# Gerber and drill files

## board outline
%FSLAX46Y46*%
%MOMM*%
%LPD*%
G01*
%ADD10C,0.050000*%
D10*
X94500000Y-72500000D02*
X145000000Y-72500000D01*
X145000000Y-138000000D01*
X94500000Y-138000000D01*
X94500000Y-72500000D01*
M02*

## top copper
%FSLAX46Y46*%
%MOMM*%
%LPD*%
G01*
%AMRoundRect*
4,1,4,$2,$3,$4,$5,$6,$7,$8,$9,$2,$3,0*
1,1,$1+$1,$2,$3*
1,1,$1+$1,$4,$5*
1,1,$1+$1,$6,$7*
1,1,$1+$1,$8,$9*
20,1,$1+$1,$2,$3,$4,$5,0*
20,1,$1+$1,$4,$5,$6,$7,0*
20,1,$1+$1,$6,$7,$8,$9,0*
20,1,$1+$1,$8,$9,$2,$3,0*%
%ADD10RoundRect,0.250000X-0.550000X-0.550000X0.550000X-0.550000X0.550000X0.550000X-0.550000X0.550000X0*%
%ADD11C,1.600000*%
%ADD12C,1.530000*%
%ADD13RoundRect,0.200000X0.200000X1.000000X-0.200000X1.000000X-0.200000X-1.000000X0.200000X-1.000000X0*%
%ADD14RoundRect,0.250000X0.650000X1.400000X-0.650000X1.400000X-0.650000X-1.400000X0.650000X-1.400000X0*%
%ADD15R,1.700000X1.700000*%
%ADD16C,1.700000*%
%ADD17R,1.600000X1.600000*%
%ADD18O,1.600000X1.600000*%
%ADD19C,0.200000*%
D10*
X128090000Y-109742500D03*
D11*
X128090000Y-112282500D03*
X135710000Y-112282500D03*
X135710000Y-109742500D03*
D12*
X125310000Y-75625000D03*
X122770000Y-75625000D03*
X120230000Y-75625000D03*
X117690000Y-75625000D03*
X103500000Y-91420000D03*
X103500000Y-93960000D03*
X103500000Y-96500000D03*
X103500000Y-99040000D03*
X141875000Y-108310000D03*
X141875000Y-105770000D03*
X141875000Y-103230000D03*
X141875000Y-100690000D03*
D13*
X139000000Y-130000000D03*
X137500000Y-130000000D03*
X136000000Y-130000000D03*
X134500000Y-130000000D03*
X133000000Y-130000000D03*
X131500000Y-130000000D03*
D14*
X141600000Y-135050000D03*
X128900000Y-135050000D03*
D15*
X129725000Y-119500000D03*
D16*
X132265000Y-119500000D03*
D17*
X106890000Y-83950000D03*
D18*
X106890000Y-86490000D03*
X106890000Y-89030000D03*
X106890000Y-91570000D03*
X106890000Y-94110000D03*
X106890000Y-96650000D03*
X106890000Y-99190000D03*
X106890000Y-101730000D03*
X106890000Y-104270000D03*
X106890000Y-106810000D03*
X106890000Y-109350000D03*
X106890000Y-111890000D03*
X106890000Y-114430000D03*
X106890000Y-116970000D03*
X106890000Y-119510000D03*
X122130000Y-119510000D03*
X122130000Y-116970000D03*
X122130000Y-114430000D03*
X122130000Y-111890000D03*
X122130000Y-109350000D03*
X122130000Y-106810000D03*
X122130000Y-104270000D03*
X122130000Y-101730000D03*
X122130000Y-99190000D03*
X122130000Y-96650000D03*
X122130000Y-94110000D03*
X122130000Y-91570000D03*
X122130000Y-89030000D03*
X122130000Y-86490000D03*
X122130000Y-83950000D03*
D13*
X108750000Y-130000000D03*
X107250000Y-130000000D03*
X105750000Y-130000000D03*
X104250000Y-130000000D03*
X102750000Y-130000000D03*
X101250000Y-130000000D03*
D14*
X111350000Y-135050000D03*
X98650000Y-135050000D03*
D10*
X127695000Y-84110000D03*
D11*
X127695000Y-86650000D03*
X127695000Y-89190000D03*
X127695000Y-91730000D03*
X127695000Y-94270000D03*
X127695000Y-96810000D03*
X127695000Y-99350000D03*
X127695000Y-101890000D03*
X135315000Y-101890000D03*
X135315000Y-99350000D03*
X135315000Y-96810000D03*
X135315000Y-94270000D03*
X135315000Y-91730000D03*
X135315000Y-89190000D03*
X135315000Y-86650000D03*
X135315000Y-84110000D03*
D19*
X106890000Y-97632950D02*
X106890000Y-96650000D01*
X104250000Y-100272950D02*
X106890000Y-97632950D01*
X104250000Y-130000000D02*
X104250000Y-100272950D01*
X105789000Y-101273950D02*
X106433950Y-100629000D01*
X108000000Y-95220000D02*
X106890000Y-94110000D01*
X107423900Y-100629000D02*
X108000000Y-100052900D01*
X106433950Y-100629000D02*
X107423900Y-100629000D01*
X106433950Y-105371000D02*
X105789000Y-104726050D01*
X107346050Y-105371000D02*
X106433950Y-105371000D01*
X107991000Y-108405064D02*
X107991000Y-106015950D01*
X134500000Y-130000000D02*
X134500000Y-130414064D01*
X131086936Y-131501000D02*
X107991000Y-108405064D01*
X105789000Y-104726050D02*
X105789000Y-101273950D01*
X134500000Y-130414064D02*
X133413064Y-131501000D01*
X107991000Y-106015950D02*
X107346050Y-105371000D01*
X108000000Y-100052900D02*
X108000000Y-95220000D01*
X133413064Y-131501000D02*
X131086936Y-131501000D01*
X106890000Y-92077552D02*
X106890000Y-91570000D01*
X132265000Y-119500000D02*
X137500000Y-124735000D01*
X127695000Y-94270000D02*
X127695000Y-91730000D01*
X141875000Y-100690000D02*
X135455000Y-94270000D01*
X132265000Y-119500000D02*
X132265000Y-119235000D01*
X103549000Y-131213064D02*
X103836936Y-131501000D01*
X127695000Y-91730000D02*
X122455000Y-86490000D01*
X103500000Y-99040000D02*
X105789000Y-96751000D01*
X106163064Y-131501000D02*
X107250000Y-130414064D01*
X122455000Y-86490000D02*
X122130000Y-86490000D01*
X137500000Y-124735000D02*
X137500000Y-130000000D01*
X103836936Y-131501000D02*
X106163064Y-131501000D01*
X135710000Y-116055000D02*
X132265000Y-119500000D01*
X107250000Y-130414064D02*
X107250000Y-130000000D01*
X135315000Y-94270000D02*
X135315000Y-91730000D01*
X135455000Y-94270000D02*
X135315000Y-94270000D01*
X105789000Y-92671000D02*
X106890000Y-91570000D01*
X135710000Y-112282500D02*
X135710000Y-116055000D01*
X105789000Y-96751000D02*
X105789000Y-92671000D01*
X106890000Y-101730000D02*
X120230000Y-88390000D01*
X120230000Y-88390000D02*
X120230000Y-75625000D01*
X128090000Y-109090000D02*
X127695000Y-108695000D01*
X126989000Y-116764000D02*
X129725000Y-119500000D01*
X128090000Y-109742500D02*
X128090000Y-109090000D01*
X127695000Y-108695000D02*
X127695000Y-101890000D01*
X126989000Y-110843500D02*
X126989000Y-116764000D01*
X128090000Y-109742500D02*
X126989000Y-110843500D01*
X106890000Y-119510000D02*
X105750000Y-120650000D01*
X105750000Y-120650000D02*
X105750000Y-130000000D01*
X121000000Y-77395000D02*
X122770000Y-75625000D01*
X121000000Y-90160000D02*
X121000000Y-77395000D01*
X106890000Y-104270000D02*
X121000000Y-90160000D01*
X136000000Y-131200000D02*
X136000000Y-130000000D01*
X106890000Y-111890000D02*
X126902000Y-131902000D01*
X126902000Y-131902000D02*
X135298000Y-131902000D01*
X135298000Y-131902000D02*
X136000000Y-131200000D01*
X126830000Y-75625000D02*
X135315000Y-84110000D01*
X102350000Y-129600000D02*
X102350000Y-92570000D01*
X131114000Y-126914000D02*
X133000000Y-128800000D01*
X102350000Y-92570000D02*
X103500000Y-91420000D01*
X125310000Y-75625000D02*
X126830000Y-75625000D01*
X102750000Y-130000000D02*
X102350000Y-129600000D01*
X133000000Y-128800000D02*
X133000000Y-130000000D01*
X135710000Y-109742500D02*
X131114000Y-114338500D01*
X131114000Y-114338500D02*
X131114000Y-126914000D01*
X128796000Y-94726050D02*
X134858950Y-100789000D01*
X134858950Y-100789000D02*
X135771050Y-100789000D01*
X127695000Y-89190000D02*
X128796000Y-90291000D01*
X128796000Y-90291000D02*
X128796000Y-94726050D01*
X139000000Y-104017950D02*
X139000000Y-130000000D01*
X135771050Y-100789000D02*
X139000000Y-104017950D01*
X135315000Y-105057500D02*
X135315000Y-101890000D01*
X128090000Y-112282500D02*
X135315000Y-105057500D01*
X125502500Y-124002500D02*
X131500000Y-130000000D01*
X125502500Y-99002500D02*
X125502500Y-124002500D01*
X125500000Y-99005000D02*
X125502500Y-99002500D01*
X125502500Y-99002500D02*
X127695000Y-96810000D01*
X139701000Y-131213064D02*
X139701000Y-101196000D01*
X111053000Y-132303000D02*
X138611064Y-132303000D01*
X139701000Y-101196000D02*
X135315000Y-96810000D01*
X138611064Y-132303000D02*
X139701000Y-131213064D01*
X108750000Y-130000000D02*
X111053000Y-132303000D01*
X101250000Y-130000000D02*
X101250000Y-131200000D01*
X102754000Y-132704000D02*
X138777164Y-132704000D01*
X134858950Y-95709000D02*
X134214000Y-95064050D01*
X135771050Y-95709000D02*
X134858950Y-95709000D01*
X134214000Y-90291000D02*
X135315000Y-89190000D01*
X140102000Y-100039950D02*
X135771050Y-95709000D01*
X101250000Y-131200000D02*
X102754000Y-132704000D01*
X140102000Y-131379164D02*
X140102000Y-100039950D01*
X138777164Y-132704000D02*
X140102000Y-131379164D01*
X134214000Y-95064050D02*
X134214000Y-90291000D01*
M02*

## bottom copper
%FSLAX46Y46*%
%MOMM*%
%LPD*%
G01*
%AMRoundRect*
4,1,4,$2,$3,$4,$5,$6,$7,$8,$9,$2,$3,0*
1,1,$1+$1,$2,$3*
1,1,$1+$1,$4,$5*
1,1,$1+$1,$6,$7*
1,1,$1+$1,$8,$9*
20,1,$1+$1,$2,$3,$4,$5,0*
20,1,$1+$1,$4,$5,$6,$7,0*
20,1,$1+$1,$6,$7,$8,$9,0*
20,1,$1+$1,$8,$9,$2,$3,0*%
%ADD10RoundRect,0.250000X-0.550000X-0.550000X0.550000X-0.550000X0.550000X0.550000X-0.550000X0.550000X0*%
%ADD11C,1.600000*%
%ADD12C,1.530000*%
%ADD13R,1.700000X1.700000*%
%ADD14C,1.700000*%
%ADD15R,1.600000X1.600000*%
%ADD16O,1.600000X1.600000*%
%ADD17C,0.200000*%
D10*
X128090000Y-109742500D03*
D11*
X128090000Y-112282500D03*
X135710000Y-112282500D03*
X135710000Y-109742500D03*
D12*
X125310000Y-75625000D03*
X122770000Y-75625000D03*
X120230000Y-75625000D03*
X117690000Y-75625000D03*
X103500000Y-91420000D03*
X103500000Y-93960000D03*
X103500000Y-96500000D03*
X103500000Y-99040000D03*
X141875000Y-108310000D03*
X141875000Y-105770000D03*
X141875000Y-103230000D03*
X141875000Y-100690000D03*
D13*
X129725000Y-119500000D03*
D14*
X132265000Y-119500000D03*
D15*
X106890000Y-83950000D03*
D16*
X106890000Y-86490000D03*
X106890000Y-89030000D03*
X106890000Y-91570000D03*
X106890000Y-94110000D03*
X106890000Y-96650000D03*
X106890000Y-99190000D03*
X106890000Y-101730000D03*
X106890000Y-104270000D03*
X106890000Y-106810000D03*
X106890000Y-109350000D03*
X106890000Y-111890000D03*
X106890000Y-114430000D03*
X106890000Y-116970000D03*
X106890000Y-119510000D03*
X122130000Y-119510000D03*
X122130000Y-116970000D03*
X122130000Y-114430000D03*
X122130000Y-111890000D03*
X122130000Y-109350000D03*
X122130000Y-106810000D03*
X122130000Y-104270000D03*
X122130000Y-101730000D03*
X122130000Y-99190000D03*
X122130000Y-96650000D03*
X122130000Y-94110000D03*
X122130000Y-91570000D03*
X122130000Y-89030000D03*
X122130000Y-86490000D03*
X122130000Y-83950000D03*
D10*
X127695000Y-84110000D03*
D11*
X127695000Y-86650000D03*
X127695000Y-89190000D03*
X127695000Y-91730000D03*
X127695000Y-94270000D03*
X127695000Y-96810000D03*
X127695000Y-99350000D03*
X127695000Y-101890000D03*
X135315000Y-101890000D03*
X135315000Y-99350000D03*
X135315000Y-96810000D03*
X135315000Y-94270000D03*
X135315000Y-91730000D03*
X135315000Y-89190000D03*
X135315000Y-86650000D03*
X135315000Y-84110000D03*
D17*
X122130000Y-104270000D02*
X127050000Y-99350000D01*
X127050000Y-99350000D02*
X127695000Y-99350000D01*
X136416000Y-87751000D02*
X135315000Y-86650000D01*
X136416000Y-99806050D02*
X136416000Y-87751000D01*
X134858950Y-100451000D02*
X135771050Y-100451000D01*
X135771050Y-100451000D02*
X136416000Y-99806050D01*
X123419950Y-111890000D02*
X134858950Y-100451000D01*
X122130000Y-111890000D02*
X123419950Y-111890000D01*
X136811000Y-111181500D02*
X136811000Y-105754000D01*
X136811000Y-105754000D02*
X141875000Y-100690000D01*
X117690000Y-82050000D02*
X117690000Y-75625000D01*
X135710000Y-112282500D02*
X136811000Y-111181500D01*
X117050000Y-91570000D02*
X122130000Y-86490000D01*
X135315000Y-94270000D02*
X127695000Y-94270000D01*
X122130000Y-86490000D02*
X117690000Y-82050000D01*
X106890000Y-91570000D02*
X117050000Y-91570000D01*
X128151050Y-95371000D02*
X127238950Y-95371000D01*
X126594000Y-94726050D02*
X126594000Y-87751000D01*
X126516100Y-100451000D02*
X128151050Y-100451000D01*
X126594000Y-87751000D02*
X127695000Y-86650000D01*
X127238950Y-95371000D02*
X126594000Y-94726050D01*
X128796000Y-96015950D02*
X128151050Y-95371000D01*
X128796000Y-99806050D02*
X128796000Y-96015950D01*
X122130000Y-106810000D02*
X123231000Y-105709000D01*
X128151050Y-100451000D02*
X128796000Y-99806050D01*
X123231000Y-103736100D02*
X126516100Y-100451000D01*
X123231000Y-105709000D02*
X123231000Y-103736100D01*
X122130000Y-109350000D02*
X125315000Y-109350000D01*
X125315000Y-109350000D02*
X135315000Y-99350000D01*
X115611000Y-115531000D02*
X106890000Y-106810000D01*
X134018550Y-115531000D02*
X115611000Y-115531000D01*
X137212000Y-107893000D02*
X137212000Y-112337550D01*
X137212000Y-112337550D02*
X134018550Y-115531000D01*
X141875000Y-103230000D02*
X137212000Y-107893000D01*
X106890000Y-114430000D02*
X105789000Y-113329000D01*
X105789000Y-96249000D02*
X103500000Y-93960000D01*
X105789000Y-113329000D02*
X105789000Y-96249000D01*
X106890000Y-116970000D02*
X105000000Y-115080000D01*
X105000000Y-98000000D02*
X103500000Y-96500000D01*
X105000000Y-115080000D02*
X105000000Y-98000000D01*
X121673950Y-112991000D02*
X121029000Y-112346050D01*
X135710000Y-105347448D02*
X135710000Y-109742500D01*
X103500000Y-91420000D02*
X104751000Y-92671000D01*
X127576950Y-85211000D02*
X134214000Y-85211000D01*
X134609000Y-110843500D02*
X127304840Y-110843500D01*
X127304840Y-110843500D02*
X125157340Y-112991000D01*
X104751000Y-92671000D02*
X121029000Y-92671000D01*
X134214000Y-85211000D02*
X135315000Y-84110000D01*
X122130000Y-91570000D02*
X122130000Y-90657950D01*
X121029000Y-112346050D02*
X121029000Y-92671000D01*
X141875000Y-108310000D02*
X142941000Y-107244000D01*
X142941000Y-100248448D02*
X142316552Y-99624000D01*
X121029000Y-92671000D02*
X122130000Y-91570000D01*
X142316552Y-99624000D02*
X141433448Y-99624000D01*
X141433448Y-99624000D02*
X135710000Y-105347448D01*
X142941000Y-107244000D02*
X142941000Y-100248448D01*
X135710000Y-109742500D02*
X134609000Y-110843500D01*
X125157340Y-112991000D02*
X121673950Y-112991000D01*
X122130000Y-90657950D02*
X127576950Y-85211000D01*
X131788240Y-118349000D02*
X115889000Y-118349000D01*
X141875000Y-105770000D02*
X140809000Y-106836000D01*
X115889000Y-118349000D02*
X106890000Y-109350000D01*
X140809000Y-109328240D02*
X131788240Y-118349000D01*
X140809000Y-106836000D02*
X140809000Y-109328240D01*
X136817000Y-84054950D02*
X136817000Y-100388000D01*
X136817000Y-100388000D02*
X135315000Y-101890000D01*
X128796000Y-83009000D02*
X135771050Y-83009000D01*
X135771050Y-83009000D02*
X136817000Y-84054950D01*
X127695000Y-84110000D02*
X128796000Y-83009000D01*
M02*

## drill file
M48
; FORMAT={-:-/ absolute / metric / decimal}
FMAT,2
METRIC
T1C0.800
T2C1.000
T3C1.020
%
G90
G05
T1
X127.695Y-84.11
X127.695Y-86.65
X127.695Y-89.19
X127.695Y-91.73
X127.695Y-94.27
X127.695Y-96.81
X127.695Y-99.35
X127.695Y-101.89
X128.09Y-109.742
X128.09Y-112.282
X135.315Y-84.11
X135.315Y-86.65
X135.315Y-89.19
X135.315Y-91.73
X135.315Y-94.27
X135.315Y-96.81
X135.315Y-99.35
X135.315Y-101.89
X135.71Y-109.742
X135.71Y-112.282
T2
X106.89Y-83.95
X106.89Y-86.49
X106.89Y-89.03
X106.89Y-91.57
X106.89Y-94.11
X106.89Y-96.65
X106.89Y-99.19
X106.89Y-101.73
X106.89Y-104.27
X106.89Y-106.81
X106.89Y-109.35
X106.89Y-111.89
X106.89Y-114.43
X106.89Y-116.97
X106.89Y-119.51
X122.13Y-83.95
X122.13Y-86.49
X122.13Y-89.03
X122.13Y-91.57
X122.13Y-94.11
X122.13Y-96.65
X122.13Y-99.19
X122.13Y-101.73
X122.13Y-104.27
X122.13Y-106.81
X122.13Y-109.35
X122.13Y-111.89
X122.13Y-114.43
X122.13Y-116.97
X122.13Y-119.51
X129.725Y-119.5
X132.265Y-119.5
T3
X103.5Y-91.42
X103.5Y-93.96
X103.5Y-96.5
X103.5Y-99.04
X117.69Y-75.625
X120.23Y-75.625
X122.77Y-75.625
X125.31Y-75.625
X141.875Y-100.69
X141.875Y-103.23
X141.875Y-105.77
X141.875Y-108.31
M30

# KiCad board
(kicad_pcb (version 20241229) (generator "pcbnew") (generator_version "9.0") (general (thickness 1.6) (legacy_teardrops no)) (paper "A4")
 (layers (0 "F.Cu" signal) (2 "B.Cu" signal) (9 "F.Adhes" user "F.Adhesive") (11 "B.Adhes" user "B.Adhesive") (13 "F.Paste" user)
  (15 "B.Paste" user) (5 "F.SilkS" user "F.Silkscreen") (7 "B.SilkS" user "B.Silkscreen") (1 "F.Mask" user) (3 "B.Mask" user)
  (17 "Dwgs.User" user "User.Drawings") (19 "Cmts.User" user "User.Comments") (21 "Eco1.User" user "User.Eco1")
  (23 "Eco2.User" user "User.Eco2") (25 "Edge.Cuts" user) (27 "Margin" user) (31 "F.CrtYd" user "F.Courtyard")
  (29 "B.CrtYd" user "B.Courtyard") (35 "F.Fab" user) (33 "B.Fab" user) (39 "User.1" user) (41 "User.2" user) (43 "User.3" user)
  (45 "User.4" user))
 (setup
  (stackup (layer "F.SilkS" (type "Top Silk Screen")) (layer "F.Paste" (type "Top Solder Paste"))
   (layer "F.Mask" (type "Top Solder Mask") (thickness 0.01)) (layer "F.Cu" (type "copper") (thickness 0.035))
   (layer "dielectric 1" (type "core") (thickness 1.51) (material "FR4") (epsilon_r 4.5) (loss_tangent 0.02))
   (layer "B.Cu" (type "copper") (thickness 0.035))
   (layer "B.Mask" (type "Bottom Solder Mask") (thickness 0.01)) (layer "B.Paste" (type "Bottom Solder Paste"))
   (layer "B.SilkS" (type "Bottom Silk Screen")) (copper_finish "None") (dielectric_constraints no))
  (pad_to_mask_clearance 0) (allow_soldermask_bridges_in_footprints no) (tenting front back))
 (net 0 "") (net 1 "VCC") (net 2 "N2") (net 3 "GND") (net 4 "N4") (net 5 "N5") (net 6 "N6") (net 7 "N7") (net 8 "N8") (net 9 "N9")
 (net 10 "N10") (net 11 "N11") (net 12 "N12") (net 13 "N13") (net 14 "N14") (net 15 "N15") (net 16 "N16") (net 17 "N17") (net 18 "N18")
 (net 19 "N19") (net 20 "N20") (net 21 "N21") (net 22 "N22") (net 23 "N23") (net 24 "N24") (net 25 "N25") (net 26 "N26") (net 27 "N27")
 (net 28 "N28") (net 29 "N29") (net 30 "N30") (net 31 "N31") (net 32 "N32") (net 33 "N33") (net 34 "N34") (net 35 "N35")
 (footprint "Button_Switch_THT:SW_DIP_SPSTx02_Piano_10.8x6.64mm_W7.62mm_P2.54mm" (layer "F.Cu") (at 128.09 109.7425)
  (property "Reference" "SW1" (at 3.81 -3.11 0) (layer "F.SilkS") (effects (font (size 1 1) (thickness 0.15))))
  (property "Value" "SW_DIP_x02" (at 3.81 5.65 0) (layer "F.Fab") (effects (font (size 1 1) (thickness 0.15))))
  (pad "1" thru_hole roundrect (at 0 0) (size 1.6 1.6) (drill 0.8) (layers "*.Cu" "*.Mask") (remove_unused_layers no)
   (roundrect_rratio 0.15625) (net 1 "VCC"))
  (pad "2" thru_hole circle (at 0 2.54) (size 1.6 1.6) (drill 0.8) (layers "*.Cu" "*.Mask") (remove_unused_layers no) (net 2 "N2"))
  (pad "3" thru_hole circle (at 7.62 2.54) (size 1.6 1.6) (drill 0.8) (layers "*.Cu" "*.Mask") (remove_unused_layers no) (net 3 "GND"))
  (pad "4" thru_hole circle (at 7.62 0) (size 1.6 1.6) (drill 0.8) (layers "*.Cu" "*.Mask") (remove_unused_layers no) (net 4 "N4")))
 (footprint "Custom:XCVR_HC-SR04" (layer "F.Cu") (at 121.5 75.625 180)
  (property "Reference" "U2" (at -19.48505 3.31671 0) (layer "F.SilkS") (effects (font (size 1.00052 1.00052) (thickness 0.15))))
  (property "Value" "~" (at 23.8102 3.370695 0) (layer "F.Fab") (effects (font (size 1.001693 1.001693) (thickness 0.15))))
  (pad "1" thru_hole circle (at -3.81 0 180) (size 1.53 1.53) (drill 1.02) (layers "*.Cu" "*.Mask") (remove_unused_layers no) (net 4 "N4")
   (solder_mask_margin 0.102))
  (pad "2" thru_hole circle (at -1.27 0 180) (size 1.53 1.53) (drill 1.02) (layers "*.Cu" "*.Mask") (remove_unused_layers no) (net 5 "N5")
   (solder_mask_margin 0.102))
  (pad "3" thru_hole circle (at 1.27 0 180) (size 1.53 1.53) (drill 1.02) (layers "*.Cu" "*.Mask") (remove_unused_layers no) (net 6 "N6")
   (solder_mask_margin 0.102))
  (pad "4" thru_hole circle (at 3.81 0 180) (size 1.53 1.53) (drill 1.02) (layers "*.Cu" "*.Mask") (remove_unused_layers no) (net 3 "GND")
   (solder_mask_margin 0.102)))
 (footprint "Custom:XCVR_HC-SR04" (layer "F.Cu") (at 103.5 95.23 -90)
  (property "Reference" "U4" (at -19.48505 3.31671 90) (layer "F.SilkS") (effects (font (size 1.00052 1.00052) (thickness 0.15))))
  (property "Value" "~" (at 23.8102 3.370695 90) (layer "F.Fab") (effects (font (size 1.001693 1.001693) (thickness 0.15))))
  (pad "1" thru_hole circle (at -3.81 0 270) (size 1.53 1.53) (drill 1.02) (layers "*.Cu" "*.Mask") (remove_unused_layers no) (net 4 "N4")
   (solder_mask_margin 0.102))
  (pad "2" thru_hole circle (at -1.27 0 270) (size 1.53 1.53) (drill 1.02) (layers "*.Cu" "*.Mask") (remove_unused_layers no) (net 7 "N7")
   (solder_mask_margin 0.102))
  (pad "3" thru_hole circle (at 1.27 0 270) (size 1.53 1.53) (drill 1.02) (layers "*.Cu" "*.Mask") (remove_unused_layers no) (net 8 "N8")
   (solder_mask_margin 0.102))
  (pad "4" thru_hole circle (at 3.81 0 270) (size 1.53 1.53) (drill 1.02) (layers "*.Cu" "*.Mask") (remove_unused_layers no) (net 3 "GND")
   (solder_mask_margin 0.102)))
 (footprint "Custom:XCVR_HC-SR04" (layer "F.Cu") (at 141.875 104.5 90)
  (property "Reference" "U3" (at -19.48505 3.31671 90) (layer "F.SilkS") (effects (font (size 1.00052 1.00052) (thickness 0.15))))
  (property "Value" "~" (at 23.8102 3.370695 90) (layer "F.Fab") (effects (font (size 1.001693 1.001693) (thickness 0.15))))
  (pad "1" thru_hole circle (at -3.81 0 90) (size 1.53 1.53) (drill 1.02) (layers "*.Cu" "*.Mask") (remove_unused_layers no) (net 4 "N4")
   (solder_mask_margin 0.102))
  (pad "2" thru_hole circle (at -1.27 0 90) (size 1.53 1.53) (drill 1.02) (layers "*.Cu" "*.Mask") (remove_unused_layers no) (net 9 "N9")
   (solder_mask_margin 0.102))
  (pad "3" thru_hole circle (at 1.27 0 90) (size 1.53 1.53) (drill 1.02) (layers "*.Cu" "*.Mask") (remove_unused_layers no) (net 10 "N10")
   (solder_mask_margin 0.102))
  (pad "4" thru_hole circle (at 3.81 0 90) (size 1.53 1.53) (drill 1.02) (layers "*.Cu" "*.Mask") (remove_unused_layers no) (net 3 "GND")
   (solder_mask_margin 0.102)))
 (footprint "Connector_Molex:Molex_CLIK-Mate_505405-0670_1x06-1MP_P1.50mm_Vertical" (layer "F.Cu") (at 135.25 132.75 180)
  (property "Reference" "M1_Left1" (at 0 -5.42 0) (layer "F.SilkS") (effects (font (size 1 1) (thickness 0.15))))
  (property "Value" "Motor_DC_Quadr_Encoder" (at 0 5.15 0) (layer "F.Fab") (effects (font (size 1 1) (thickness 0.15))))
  (pad "1" smd roundrect (at -3.75 2.75 180) (size 0.8 2.4) (layers "F.Cu" "F.Mask" "F.Paste") (roundrect_rratio 0.25) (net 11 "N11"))
  (pad "2" smd roundrect (at -2.25 2.75 180) (size 0.8 2.4) (layers "F.Cu" "F.Mask" "F.Paste") (roundrect_rratio 0.25) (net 3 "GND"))
  (pad "3" smd roundrect (at -0.75 2.75 180) (size 0.8 2.4) (layers "F.Cu" "F.Mask" "F.Paste") (roundrect_rratio 0.25) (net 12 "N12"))
  (pad "4" smd roundrect (at 0.75 2.75 180) (size 0.8 2.4) (layers "F.Cu" "F.Mask" "F.Paste") (roundrect_rratio 0.25) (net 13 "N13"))
  (pad "5" smd roundrect (at 2.25 2.75 180) (size 0.8 2.4) (layers "F.Cu" "F.Mask" "F.Paste") (roundrect_rratio 0.25) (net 4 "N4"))
  (pad "6" smd roundrect (at 3.75 2.75 180) (size 0.8 2.4) (layers "F.Cu" "F.Mask" "F.Paste") (roundrect_rratio 0.25) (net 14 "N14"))
  (pad "MP" smd roundrect (at -6.35 -2.3 180) (size 1.8 3.3) (layers "F.Cu" "F.Mask" "F.Paste") (roundrect_rratio 0.138889))
  (pad "MP" smd roundrect (at 6.35 -2.3 180) (size 1.8 3.3) (layers "F.Cu" "F.Mask" "F.Paste") (roundrect_rratio 0.138889)))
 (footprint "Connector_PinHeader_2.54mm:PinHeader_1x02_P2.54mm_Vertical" (layer "F.Cu") (at 129.725 119.5 90)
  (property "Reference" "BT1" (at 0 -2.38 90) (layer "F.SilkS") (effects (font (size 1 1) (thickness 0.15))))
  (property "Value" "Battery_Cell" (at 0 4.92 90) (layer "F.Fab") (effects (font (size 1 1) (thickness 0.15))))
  (pad "1" thru_hole rect (at 0 0 90) (size 1.7 1.7) (drill 1) (layers "*.Cu" "*.Mask") (remove_unused_layers no) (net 1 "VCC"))
  (pad "2" thru_hole circle (at 0 2.54 90) (size 1.7 1.7) (drill 1) (layers "*.Cu" "*.Mask") (remove_unused_layers no) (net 3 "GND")))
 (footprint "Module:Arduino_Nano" (layer "F.Cu") (at 106.89 83.95)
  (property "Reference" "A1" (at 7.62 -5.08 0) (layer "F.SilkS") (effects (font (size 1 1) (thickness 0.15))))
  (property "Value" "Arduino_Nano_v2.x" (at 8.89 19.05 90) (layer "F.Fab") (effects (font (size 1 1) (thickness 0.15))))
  (pad "1" thru_hole rect (at 0 0) (size 1.6 1.6) (drill 1) (layers "*.Cu" "*.Mask") (remove_unused_layers no) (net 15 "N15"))
  (pad "2" thru_hole oval (at 0 2.54) (size 1.6 1.6) (drill 1) (layers "*.Cu" "*.Mask") (remove_unused_layers no) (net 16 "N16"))
  (pad "3" thru_hole oval (at 0 5.08) (size 1.6 1.6) (drill 1) (layers "*.Cu" "*.Mask") (remove_unused_layers no) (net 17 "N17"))
  (pad "4" thru_hole oval (at 0 7.62) (size 1.6 1.6) (drill 1) (layers "*.Cu" "*.Mask") (remove_unused_layers no) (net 3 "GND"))
  (pad "5" thru_hole oval (at 0 10.16) (size 1.6 1.6) (drill 1) (layers "*.Cu" "*.Mask") (remove_unused_layers no) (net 13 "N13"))
  (pad "6" thru_hole oval (at 0 12.7) (size 1.6 1.6) (drill 1) (layers "*.Cu" "*.Mask") (remove_unused_layers no) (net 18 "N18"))
  (pad "7" thru_hole oval (at 0 15.24) (size 1.6 1.6) (drill 1) (layers "*.Cu" "*.Mask") (remove_unused_layers no) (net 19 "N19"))
  (pad "8" thru_hole oval (at 0 17.78) (size 1.6 1.6) (drill 1) (layers "*.Cu" "*.Mask") (remove_unused_layers no) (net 6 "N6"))
  (pad "9" thru_hole oval (at 0 20.32) (size 1.6 1.6) (drill 1) (layers "*.Cu" "*.Mask") (remove_unused_layers no) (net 5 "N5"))
  (pad "10" thru_hole oval (at 0 22.86) (size 1.6 1.6) (drill 1) (layers "*.Cu" "*.Mask") (remove_unused_layers no) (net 10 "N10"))
  (pad "11" thru_hole oval (at 0 25.4) (size 1.6 1.6) (drill 1) (layers "*.Cu" "*.Mask") (remove_unused_layers no) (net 9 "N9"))
  (pad "12" thru_hole oval (at 0 27.94) (size 1.6 1.6) (drill 1) (layers "*.Cu" "*.Mask") (remove_unused_layers no) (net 12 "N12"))
  (pad "13" thru_hole oval (at 0 30.48) (size 1.6 1.6) (drill 1) (layers "*.Cu" "*.Mask") (remove_unused_layers no) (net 7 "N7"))
  (pad "14" thru_hole oval (at 0 33.02) (size 1.6 1.6) (drill 1) (layers "*.Cu" "*.Mask") (remove_unused_layers no) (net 8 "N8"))
  (pad "15" thru_hole oval (at 0 35.56) (size 1.6 1.6) (drill 1) (layers "*.Cu" "*.Mask") (remove_unused_layers no) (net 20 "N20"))
  (pad "16" thru_hole oval (at 15.24 35.56) (size 1.6 1.6) (drill 1) (layers "*.Cu" "*.Mask") (remove_unused_layers no) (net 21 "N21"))
  (pad "17" thru_hole oval (at 15.24 33.02) (size 1.6 1.6) (drill 1) (layers "*.Cu" "*.Mask") (remove_unused_layers no) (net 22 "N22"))
  (pad "18" thru_hole oval (at 15.24 30.48) (size 1.6 1.6) (drill 1) (layers "*.Cu" "*.Mask") (remove_unused_layers no) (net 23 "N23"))
  (pad "19" thru_hole oval (at 15.24 27.94) (size 1.6 1.6) (drill 1) (layers "*.Cu" "*.Mask") (remove_unused_layers no) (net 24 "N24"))
  (pad "20" thru_hole oval (at 15.24 25.4) (size 1.6 1.6) (drill 1) (layers "*.Cu" "*.Mask") (remove_unused_layers no) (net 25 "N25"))
  (pad "21" thru_hole oval (at 15.24 22.86) (size 1.6 1.6) (drill 1) (layers "*.Cu" "*.Mask") (remove_unused_layers no) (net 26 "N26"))
  (pad "22" thru_hole oval (at 15.24 20.32) (size 1.6 1.6) (drill 1) (layers "*.Cu" "*.Mask") (remove_unused_layers no) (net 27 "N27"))
  (pad "23" thru_hole oval (at 15.24 17.78) (size 1.6 1.6) (drill 1) (layers "*.Cu" "*.Mask") (remove_unused_layers no) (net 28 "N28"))
  (pad "24" thru_hole oval (at 15.24 15.24) (size 1.6 1.6) (drill 1) (layers "*.Cu" "*.Mask") (remove_unused_layers no) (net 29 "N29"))
  (pad "25" thru_hole oval (at 15.24 12.7) (size 1.6 1.6) (drill 1) (layers "*.Cu" "*.Mask") (remove_unused_layers no) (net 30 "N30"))
  (pad "26" thru_hole oval (at 15.24 10.16) (size 1.6 1.6) (drill 1) (layers "*.Cu" "*.Mask") (remove_unused_layers no) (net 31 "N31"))
  (pad "27" thru_hole oval (at 15.24 7.62) (size 1.6 1.6) (drill 1) (layers "*.Cu" "*.Mask") (remove_unused_layers no) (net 4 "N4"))
  (pad "28" thru_hole oval (at 15.24 5.08) (size 1.6 1.6) (drill 1) (layers "*.Cu" "*.Mask") (remove_unused_layers no) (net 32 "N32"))
  (pad "29" thru_hole oval (at 15.24 2.54) (size 1.6 1.6) (drill 1) (layers "*.Cu" "*.Mask") (remove_unused_layers no) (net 3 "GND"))
  (pad "30" thru_hole oval (at 15.24 0) (size 1.6 1.6) (drill 1) (layers "*.Cu" "*.Mask") (remove_unused_layers no) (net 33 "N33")))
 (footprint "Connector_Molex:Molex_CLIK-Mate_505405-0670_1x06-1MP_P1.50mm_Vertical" (layer "F.Cu") (at 105 132.75 180)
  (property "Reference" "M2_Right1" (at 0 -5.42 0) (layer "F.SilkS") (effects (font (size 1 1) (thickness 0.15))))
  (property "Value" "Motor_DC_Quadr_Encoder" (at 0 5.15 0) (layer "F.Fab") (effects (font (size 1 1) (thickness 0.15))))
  (pad "1" smd roundrect (at -3.75 2.75 180) (size 0.8 2.4) (layers "F.Cu" "F.Mask" "F.Paste") (roundrect_rratio 0.25) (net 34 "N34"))
  (pad "2" smd roundrect (at -2.25 2.75 180) (size 0.8 2.4) (layers "F.Cu" "F.Mask" "F.Paste") (roundrect_rratio 0.25) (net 3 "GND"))
  (pad "3" smd roundrect (at -0.75 2.75 180) (size 0.8 2.4) (layers "F.Cu" "F.Mask" "F.Paste") (roundrect_rratio 0.25) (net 20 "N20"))
  (pad "4" smd roundrect (at 0.75 2.75 180) (size 0.8 2.4) (layers "F.Cu" "F.Mask" "F.Paste") (roundrect_rratio 0.25) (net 18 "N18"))
  (pad "5" smd roundrect (at 2.25 2.75 180) (size 0.8 2.4) (layers "F.Cu" "F.Mask" "F.Paste") (roundrect_rratio 0.25) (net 4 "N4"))
  (pad "6" smd roundrect (at 3.75 2.75 180) (size 0.8 2.4) (layers "F.Cu" "F.Mask" "F.Paste") (roundrect_rratio 0.25) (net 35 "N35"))
  (pad "MP" smd roundrect (at -6.35 -2.3 180) (size 1.8 3.3) (layers "F.Cu" "F.Mask" "F.Paste") (roundrect_rratio 0.138889))
  (pad "MP" smd roundrect (at 6.35 -2.3 180) (size 1.8 3.3) (layers "F.Cu" "F.Mask" "F.Paste") (roundrect_rratio 0.138889)))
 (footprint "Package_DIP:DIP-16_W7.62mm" (layer "F.Cu") (at 127.695 84.11)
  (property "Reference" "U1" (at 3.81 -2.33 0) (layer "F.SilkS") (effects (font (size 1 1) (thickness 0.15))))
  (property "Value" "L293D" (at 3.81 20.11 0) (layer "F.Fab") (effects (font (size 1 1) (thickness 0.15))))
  (pad "1" thru_hole roundrect (at 0 0) (size 1.6 1.6) (drill 0.8) (layers "*.Cu" "*.Mask") (remove_unused_layers no)
   (roundrect_rratio 0.15625) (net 2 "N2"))
  (pad "2" thru_hole circle (at 0 2.54) (size 1.6 1.6) (drill 0.8) (layers "*.Cu" "*.Mask") (remove_unused_layers no) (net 26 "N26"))
  (pad "3" thru_hole circle (at 0 5.08) (size 1.6 1.6) (drill 0.8) (layers "*.Cu" "*.Mask") (remove_unused_layers no) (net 11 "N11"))
  (pad "4" thru_hole circle (at 0 7.62) (size 1.6 1.6) (drill 0.8) (layers "*.Cu" "*.Mask") (remove_unused_layers no) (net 3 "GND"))
  (pad "5" thru_hole circle (at 0 10.16) (size 1.6 1.6) (drill 0.8) (layers "*.Cu" "*.Mask") (remove_unused_layers no) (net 3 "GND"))
  (pad "6" thru_hole circle (at 0 12.7) (size 1.6 1.6) (drill 0.8) (layers "*.Cu" "*.Mask") (remove_unused_layers no) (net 14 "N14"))
  (pad "7" thru_hole circle (at 0 15.24) (size 1.6 1.6) (drill 0.8) (layers "*.Cu" "*.Mask") (remove_unused_layers no) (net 27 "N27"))
  (pad "8" thru_hole circle (at 0 17.78) (size 1.6 1.6) (drill 0.8) (layers "*.Cu" "*.Mask") (remove_unused_layers no) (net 1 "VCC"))
  (pad "9" thru_hole circle (at 7.62 17.78) (size 1.6 1.6) (drill 0.8) (layers "*.Cu" "*.Mask") (remove_unused_layers no) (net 2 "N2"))
  (pad "10" thru_hole circle (at 7.62 15.24) (size 1.6 1.6) (drill 0.8) (layers "*.Cu" "*.Mask") (remove_unused_layers no) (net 25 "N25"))
  (pad "11" thru_hole circle (at 7.62 12.7) (size 1.6 1.6) (drill 0.8) (layers "*.Cu" "*.Mask") (remove_unused_layers no) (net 34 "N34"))
  (pad "12" thru_hole circle (at 7.62 10.16) (size 1.6 1.6) (drill 0.8) (layers "*.Cu" "*.Mask") (remove_unused_layers no) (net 3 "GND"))
  (pad "13" thru_hole circle (at 7.62 7.62) (size 1.6 1.6) (drill 0.8) (layers "*.Cu" "*.Mask") (remove_unused_layers no) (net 3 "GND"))
  (pad "14" thru_hole circle (at 7.62 5.08) (size 1.6 1.6) (drill 0.8) (layers "*.Cu" "*.Mask") (remove_unused_layers no) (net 35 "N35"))
  (pad "15" thru_hole circle (at 7.62 2.54) (size 1.6 1.6) (drill 0.8) (layers "*.Cu" "*.Mask") (remove_unused_layers no) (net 24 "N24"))
  (pad "16" thru_hole circle (at 7.62 0) (size 1.6 1.6) (drill 0.8) (layers "*.Cu" "*.Mask") (remove_unused_layers no) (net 4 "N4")))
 (gr_rect (start 94.5 72.5) (end 145 138) (stroke (width 0.05) (type default)) (fill no) (layer "Edge.Cuts"))
 (segment (start 106.89 97.63295) (end 106.89 96.65) (width 0.2) (layer "F.Cu") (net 18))
 (segment (start 104.25 100.27295) (end 106.89 97.63295) (width 0.2) (layer "F.Cu") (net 18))
 (segment (start 104.25 130) (end 104.25 100.27295) (width 0.2) (layer "F.Cu") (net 18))
 (segment (start 105.789 101.27395) (end 106.43395 100.629) (width 0.2) (layer "F.Cu") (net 13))
 (segment (start 108 95.22) (end 106.89 94.11) (width 0.2) (layer "F.Cu") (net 13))
 (segment (start 107.4239 100.629) (end 108 100.0529) (width 0.2) (layer "F.Cu") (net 13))
 (segment (start 106.43395 100.629) (end 107.4239 100.629) (width 0.2) (layer "F.Cu") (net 13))
 (segment (start 106.43395 105.371) (end 105.789 104.72605) (width 0.2) (layer "F.Cu") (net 13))
 (segment (start 107.34605 105.371) (end 106.43395 105.371) (width 0.2) (layer "F.Cu") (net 13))
 (segment (start 107.991 108.405064) (end 107.991 106.01595) (width 0.2) (layer "F.Cu") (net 13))
 (segment (start 134.5 130) (end 134.5 130.414064) (width 0.2) (layer "F.Cu") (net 13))
 (segment (start 131.086936 131.501) (end 107.991 108.405064) (width 0.2) (layer "F.Cu") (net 13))
 (segment (start 105.789 104.72605) (end 105.789 101.27395) (width 0.2) (layer "F.Cu") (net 13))
 (segment (start 134.5 130.414064) (end 133.413064 131.501) (width 0.2) (layer "F.Cu") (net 13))
 (segment (start 107.991 106.01595) (end 107.34605 105.371) (width 0.2) (layer "F.Cu") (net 13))
 (segment (start 108 100.0529) (end 108 95.22) (width 0.2) (layer "F.Cu") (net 13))
 (segment (start 133.413064 131.501) (end 131.086936 131.501) (width 0.2) (layer "F.Cu") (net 13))
 (segment (start 122.13 104.27) (end 127.05 99.35) (width 0.2) (layer "B.Cu") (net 27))
 (segment (start 127.05 99.35) (end 127.695 99.35) (width 0.2) (layer "B.Cu") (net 27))
 (segment (start 136.416 87.751) (end 135.315 86.65) (width 0.2) (layer "B.Cu") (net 24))
 (segment (start 136.416 99.80605) (end 136.416 87.751) (width 0.2) (layer "B.Cu") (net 24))
 (segment (start 134.85895 100.451) (end 135.77105 100.451) (width 0.2) (layer "B.Cu") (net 24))
 (segment (start 135.77105 100.451) (end 136.416 99.80605) (width 0.2) (layer "B.Cu") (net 24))
 (segment (start 123.41995 111.89) (end 134.85895 100.451) (width 0.2) (layer "B.Cu") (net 24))
 (segment (start 122.13 111.89) (end 123.41995 111.89) (width 0.2) (layer "B.Cu") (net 24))
 (segment (start 106.89 92.077552) (end 106.89 91.57) (width 0.2) (layer "F.Cu") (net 3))
 (segment (start 132.265 119.5) (end 137.5 124.735) (width 0.2) (layer "F.Cu") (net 3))
 (segment (start 127.695 94.27) (end 127.695 91.73) (width 0.2) (layer "F.Cu") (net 3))
 (segment (start 141.875 100.69) (end 135.455 94.27) (width 0.2) (layer "F.Cu") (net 3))
 (segment (start 132.265 119.5) (end 132.265 119.235) (width 0.2) (layer "F.Cu") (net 3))
 (segment (start 103.549 131.213064) (end 103.836936 131.501) (width 0.2) (layer "F.Cu") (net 3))
 (segment (start 127.695 91.73) (end 122.455 86.49) (width 0.2) (layer "F.Cu") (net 3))
 (segment (start 103.5 99.04) (end 105.789 96.751) (width 0.2) (layer "F.Cu") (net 3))
 (segment (start 106.163064 131.501) (end 107.25 130.414064) (width 0.2) (layer "F.Cu") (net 3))
 (segment (start 122.455 86.49) (end 122.13 86.49) (width 0.2) (layer "F.Cu") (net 3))
 (segment (start 137.5 124.735) (end 137.5 130) (width 0.2) (layer "F.Cu") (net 3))
 (segment (start 103.836936 131.501) (end 106.163064 131.501) (width 0.2) (layer "F.Cu") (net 3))
 (segment (start 135.71 116.055) (end 132.265 119.5) (width 0.2) (layer "F.Cu") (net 3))
 (segment (start 107.25 130.414064) (end 107.25 130) (width 0.2) (layer "F.Cu") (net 3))
 (segment (start 135.315 94.27) (end 135.315 91.73) (width 0.2) (layer "F.Cu") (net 3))
 (segment (start 135.455 94.27) (end 135.315 94.27) (width 0.2) (layer "F.Cu") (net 3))
 (segment (start 105.789 92.671) (end 106.89 91.57) (width 0.2) (layer "F.Cu") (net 3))
 (segment (start 135.71 112.2825) (end 135.71 116.055) (width 0.2) (layer "F.Cu") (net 3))
 (segment (start 105.789 96.751) (end 105.789 92.671) (width 0.2) (layer "F.Cu") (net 3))
 (segment (start 136.811 111.1815) (end 136.811 105.754) (width 0.2) (layer "B.Cu") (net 3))
 (segment (start 136.811 105.754) (end 141.875 100.69) (width 0.2) (layer "B.Cu") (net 3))
 (segment (start 117.69 82.05) (end 117.69 75.625) (width 0.2) (layer "B.Cu") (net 3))
 (segment (start 135.71 112.2825) (end 136.811 111.1815) (width 0.2) (layer "B.Cu") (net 3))
 (segment (start 117.05 91.57) (end 122.13 86.49) (width 0.2) (layer "B.Cu") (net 3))
 (segment (start 135.315 94.27) (end 127.695 94.27) (width 0.2) (layer "B.Cu") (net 3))
 (segment (start 122.13 86.49) (end 117.69 82.05) (width 0.2) (layer "B.Cu") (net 3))
 (segment (start 106.89 91.57) (end 117.05 91.57) (width 0.2) (layer "B.Cu") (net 3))
 (segment (start 128.15105 95.371) (end 127.23895 95.371) (width 0.2) (layer "B.Cu") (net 26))
 (segment (start 126.594 94.72605) (end 126.594 87.751) (width 0.2) (layer "B.Cu") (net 26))
 (segment (start 126.5161 100.451) (end 128.15105 100.451) (width 0.2) (layer "B.Cu") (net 26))
 (segment (start 126.594 87.751) (end 127.695 86.65) (width 0.2) (layer "B.Cu") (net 26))
 (segment (start 127.23895 95.371) (end 126.594 94.72605) (width 0.2) (layer "B.Cu") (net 26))
 (segment (start 128.796 96.01595) (end 128.15105 95.371) (width 0.2) (layer "B.Cu") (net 26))
 (segment (start 128.796 99.80605) (end 128.796 96.01595) (width 0.2) (layer "B.Cu") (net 26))
 (segment (start 122.13 106.81) (end 123.231 105.709) (width 0.2) (layer "B.Cu") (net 26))
 (segment (start 128.15105 100.451) (end 128.796 99.80605) (width 0.2) (layer "B.Cu") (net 26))
 (segment (start 123.231 103.7361) (end 126.5161 100.451) (width 0.2) (layer "B.Cu") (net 26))
 (segment (start 123.231 105.709) (end 123.231 103.7361) (width 0.2) (layer "B.Cu") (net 26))
 (segment (start 122.13 109.35) (end 125.315 109.35) (width 0.2) (layer "B.Cu") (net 25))
 (segment (start 125.315 109.35) (end 135.315 99.35) (width 0.2) (layer "B.Cu") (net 25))
 (segment (start 106.89 101.73) (end 120.23 88.39) (width 0.2) (layer "F.Cu") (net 6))
 (segment (start 120.23 88.39) (end 120.23 75.625) (width 0.2) (layer "F.Cu") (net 6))
 (segment (start 128.09 109.09) (end 127.695 108.695) (width 0.2) (layer "F.Cu") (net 1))
 (segment (start 126.989 116.764) (end 129.725 119.5) (width 0.2) (layer "F.Cu") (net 1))
 (segment (start 128.09 109.7425) (end 128.09 109.09) (width 0.2) (layer "F.Cu") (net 1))
 (segment (start 127.695 108.695) (end 127.695 101.89) (width 0.2) (layer "F.Cu") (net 1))
 (segment (start 126.989 110.8435) (end 126.989 116.764) (width 0.2) (layer "F.Cu") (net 1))
 (segment (start 128.09 109.7425) (end 126.989 110.8435) (width 0.2) (layer "F.Cu") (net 1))
 (segment (start 106.89 119.51) (end 105.75 120.65) (width 0.2) (layer "F.Cu") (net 20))
 (segment (start 105.75 120.65) (end 105.75 130) (width 0.2) (layer "F.Cu") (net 20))
 (segment (start 121 77.395) (end 122.77 75.625) (width 0.2) (layer "F.Cu") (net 5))
 (segment (start 121 90.16) (end 121 77.395) (width 0.2) (layer "F.Cu") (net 5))
 (segment (start 106.89 104.27) (end 121 90.16) (width 0.2) (layer "F.Cu") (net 5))
 (segment (start 115.611 115.531) (end 106.89 106.81) (width 0.2) (layer "B.Cu") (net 10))
 (segment (start 134.01855 115.531) (end 115.611 115.531) (width 0.2) (layer "B.Cu") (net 10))
 (segment (start 137.212 107.893) (end 137.212 112.33755) (width 0.2) (layer "B.Cu") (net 10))
 (segment (start 137.212 112.33755) (end 134.01855 115.531) (width 0.2) (layer "B.Cu") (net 10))
 (segment (start 141.875 103.23) (end 137.212 107.893) (width 0.2) (layer "B.Cu") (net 10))
 (segment (start 106.89 114.43) (end 105.789 113.329) (width 0.2) (layer "B.Cu") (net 7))
 (segment (start 105.789 96.249) (end 103.5 93.96) (width 0.2) (layer "B.Cu") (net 7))
 (segment (start 105.789 113.329) (end 105.789 96.249) (width 0.2) (layer "B.Cu") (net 7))
 (segment (start 106.89 116.97) (end 105 115.08) (width 0.2) (layer "B.Cu") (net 8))
 (segment (start 105 98) (end 103.5 96.5) (width 0.2) (layer "B.Cu") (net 8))
 (segment (start 105 115.08) (end 105 98) (width 0.2) (layer "B.Cu") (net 8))
 (segment (start 136 131.2) (end 136 130) (width 0.2) (layer "F.Cu") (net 12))
 (segment (start 106.89 111.89) (end 126.902 131.902) (width 0.2) (layer "F.Cu") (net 12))
 (segment (start 126.902 131.902) (end 135.298 131.902) (width 0.2) (layer "F.Cu") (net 12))
 (segment (start 135.298 131.902) (end 136 131.2) (width 0.2) (layer "F.Cu") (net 12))
 (segment (start 126.83 75.625) (end 135.315 84.11) (width 0.2) (layer "F.Cu") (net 4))
 (segment (start 102.35 129.6) (end 102.35 92.57) (width 0.2) (layer "F.Cu") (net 4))
 (segment (start 131.114 126.914) (end 133 128.8) (width 0.2) (layer "F.Cu") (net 4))
 (segment (start 102.35 92.57) (end 103.5 91.42) (width 0.2) (layer "F.Cu") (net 4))
 (segment (start 125.31 75.625) (end 126.83 75.625) (width 0.2) (layer "F.Cu") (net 4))
 (segment (start 102.75 130) (end 102.35 129.6) (width 0.2) (layer "F.Cu") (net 4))
 (segment (start 133 128.8) (end 133 130) (width 0.2) (layer "F.Cu") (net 4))
 (segment (start 135.71 109.7425) (end 131.114 114.3385) (width 0.2) (layer "F.Cu") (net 4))
 (segment (start 131.114 114.3385) (end 131.114 126.914) (width 0.2) (layer "F.Cu") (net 4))
 (segment (start 121.67395 112.991) (end 121.029 112.34605) (width 0.2) (layer "B.Cu") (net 4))
 (segment (start 135.71 105.347448) (end 135.71 109.7425) (width 0.2) (layer "B.Cu") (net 4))
 (segment (start 103.5 91.42) (end 104.751 92.671) (width 0.2) (layer "B.Cu") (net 4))
 (segment (start 127.57695 85.211) (end 134.214 85.211) (width 0.2) (layer "B.Cu") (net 4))
 (segment (start 134.609 110.8435) (end 127.30484 110.8435) (width 0.2) (layer "B.Cu") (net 4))
 (segment (start 127.30484 110.8435) (end 125.15734 112.991) (width 0.2) (layer "B.Cu") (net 4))
 (segment (start 104.751 92.671) (end 121.029 92.671) (width 0.2) (layer "B.Cu") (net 4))
 (segment (start 134.214 85.211) (end 135.315 84.11) (width 0.2) (layer "B.Cu") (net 4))
 (segment (start 122.13 91.57) (end 122.13 90.65795) (width 0.2) (layer "B.Cu") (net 4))
 (segment (start 121.029 112.34605) (end 121.029 92.671) (width 0.2) (layer "B.Cu") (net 4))
 (segment (start 141.875 108.31) (end 142.941 107.244) (width 0.2) (layer "B.Cu") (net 4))
 (segment (start 142.941 100.248448) (end 142.316552 99.624) (width 0.2) (layer "B.Cu") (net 4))
 (segment (start 121.029 92.671) (end 122.13 91.57) (width 0.2) (layer "B.Cu") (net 4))
 (segment (start 142.316552 99.624) (end 141.433448 99.624) (width 0.2) (layer "B.Cu") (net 4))
 (segment (start 141.433448 99.624) (end 135.71 105.347448) (width 0.2) (layer "B.Cu") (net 4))
 (segment (start 142.941 107.244) (end 142.941 100.248448) (width 0.2) (layer "B.Cu") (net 4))
 (segment (start 135.71 109.7425) (end 134.609 110.8435) (width 0.2) (layer "B.Cu") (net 4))
 (segment (start 125.15734 112.991) (end 121.67395 112.991) (width 0.2) (layer "B.Cu") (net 4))
 (segment (start 122.13 90.65795) (end 127.57695 85.211) (width 0.2) (layer "B.Cu") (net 4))
 (segment (start 131.78824 118.349) (end 115.889 118.349) (width 0.2) (layer "B.Cu") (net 9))
 (segment (start 141.875 105.77) (end 140.809 106.836) (width 0.2) (layer "B.Cu") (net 9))
 (segment (start 115.889 118.349) (end 106.89 109.35) (width 0.2) (layer "B.Cu") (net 9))
 (segment (start 140.809 109.32824) (end 131.78824 118.349) (width 0.2) (layer "B.Cu") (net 9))
 (segment (start 140.809 106.836) (end 140.809 109.32824) (width 0.2) (layer "B.Cu") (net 9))
 (segment (start 128.796 94.72605) (end 134.85895 100.789) (width 0.2) (layer "F.Cu") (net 11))
 (segment (start 134.85895 100.789) (end 135.77105 100.789) (width 0.2) (layer "F.Cu") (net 11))
 (segment (start 127.695 89.19) (end 128.796 90.291) (width 0.2) (layer "F.Cu") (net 11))
 (segment (start 128.796 90.291) (end 128.796 94.72605) (width 0.2) (layer "F.Cu") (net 11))
 (segment (start 139 104.01795) (end 139 130) (width 0.2) (layer "F.Cu") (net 11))
 (segment (start 135.77105 100.789) (end 139 104.01795) (width 0.2) (layer "F.Cu") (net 11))
 (segment (start 135.315 105.0575) (end 135.315 101.89) (width 0.2) (layer "F.Cu") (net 2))
 (segment (start 128.09 112.2825) (end 135.315 105.0575) (width 0.2) (layer "F.Cu") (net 2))
 (segment (start 136.817 84.05495) (end 136.817 100.388) (width 0.2) (layer "B.Cu") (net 2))
 (segment (start 136.817 100.388) (end 135.315 101.89) (width 0.2) (layer "B.Cu") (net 2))
 (segment (start 128.796 83.009) (end 135.77105 83.009) (width 0.2) (layer "B.Cu") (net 2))
 (segment (start 135.77105 83.009) (end 136.817 84.05495) (width 0.2) (layer "B.Cu") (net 2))
 (segment (start 127.695 84.11) (end 128.796 83.009) (width 0.2) (layer "B.Cu") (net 2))
 (segment (start 125.5025 124.0025) (end 131.5 130) (width 0.2) (layer "F.Cu") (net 14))
 (segment (start 125.5025 99.0025) (end 125.5025 124.0025) (width 0.2) (layer "F.Cu") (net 14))
 (segment (start 125.5 99.005) (end 125.5025 99.0025) (width 0.2) (layer "F.Cu") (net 14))
 (segment (start 125.5025 99.0025) (end 127.695 96.81) (width 0.2) (layer "F.Cu") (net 14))
 (segment (start 139.701 131.213064) (end 139.701 101.196) (width 0.2) (layer "F.Cu") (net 34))
 (segment (start 111.053 132.303) (end 138.611064 132.303) (width 0.2) (layer "F.Cu") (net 34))
 (segment (start 139.701 101.196) (end 135.315 96.81) (width 0.2) (layer "F.Cu") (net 34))
 (segment (start 138.611064 132.303) (end 139.701 131.213064) (width 0.2) (layer "F.Cu") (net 34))
 (segment (start 108.75 130) (end 111.053 132.303) (width 0.2) (layer "F.Cu") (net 34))
 (segment (start 101.25 130) (end 101.25 131.2) (width 0.2) (layer "F.Cu") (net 35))
 (segment (start 102.754 132.704) (end 138.777164 132.704) (width 0.2) (layer "F.Cu") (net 35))
 (segment (start 134.85895 95.709) (end 134.214 95.06405) (width 0.2) (layer "F.Cu") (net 35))
 (segment (start 135.77105 95.709) (end 134.85895 95.709) (width 0.2) (layer "F.Cu") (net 35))
 (segment (start 134.214 90.291) (end 135.315 89.19) (width 0.2) (layer "F.Cu") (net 35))
 (segment (start 140.102 100.03995) (end 135.77105 95.709) (width 0.2) (layer "F.Cu") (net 35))
 (segment (start 101.25 131.2) (end 102.754 132.704) (width 0.2) (layer "F.Cu") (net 35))
 (segment (start 140.102 131.379164) (end 140.102 100.03995) (width 0.2) (layer "F.Cu") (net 35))
 (segment (start 138.777164 132.704) (end 140.102 131.379164) (width 0.2) (layer "F.Cu") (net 35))
 (segment (start 134.214 95.06405) (end 134.214 90.291) (width 0.2) (layer "F.Cu") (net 35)))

